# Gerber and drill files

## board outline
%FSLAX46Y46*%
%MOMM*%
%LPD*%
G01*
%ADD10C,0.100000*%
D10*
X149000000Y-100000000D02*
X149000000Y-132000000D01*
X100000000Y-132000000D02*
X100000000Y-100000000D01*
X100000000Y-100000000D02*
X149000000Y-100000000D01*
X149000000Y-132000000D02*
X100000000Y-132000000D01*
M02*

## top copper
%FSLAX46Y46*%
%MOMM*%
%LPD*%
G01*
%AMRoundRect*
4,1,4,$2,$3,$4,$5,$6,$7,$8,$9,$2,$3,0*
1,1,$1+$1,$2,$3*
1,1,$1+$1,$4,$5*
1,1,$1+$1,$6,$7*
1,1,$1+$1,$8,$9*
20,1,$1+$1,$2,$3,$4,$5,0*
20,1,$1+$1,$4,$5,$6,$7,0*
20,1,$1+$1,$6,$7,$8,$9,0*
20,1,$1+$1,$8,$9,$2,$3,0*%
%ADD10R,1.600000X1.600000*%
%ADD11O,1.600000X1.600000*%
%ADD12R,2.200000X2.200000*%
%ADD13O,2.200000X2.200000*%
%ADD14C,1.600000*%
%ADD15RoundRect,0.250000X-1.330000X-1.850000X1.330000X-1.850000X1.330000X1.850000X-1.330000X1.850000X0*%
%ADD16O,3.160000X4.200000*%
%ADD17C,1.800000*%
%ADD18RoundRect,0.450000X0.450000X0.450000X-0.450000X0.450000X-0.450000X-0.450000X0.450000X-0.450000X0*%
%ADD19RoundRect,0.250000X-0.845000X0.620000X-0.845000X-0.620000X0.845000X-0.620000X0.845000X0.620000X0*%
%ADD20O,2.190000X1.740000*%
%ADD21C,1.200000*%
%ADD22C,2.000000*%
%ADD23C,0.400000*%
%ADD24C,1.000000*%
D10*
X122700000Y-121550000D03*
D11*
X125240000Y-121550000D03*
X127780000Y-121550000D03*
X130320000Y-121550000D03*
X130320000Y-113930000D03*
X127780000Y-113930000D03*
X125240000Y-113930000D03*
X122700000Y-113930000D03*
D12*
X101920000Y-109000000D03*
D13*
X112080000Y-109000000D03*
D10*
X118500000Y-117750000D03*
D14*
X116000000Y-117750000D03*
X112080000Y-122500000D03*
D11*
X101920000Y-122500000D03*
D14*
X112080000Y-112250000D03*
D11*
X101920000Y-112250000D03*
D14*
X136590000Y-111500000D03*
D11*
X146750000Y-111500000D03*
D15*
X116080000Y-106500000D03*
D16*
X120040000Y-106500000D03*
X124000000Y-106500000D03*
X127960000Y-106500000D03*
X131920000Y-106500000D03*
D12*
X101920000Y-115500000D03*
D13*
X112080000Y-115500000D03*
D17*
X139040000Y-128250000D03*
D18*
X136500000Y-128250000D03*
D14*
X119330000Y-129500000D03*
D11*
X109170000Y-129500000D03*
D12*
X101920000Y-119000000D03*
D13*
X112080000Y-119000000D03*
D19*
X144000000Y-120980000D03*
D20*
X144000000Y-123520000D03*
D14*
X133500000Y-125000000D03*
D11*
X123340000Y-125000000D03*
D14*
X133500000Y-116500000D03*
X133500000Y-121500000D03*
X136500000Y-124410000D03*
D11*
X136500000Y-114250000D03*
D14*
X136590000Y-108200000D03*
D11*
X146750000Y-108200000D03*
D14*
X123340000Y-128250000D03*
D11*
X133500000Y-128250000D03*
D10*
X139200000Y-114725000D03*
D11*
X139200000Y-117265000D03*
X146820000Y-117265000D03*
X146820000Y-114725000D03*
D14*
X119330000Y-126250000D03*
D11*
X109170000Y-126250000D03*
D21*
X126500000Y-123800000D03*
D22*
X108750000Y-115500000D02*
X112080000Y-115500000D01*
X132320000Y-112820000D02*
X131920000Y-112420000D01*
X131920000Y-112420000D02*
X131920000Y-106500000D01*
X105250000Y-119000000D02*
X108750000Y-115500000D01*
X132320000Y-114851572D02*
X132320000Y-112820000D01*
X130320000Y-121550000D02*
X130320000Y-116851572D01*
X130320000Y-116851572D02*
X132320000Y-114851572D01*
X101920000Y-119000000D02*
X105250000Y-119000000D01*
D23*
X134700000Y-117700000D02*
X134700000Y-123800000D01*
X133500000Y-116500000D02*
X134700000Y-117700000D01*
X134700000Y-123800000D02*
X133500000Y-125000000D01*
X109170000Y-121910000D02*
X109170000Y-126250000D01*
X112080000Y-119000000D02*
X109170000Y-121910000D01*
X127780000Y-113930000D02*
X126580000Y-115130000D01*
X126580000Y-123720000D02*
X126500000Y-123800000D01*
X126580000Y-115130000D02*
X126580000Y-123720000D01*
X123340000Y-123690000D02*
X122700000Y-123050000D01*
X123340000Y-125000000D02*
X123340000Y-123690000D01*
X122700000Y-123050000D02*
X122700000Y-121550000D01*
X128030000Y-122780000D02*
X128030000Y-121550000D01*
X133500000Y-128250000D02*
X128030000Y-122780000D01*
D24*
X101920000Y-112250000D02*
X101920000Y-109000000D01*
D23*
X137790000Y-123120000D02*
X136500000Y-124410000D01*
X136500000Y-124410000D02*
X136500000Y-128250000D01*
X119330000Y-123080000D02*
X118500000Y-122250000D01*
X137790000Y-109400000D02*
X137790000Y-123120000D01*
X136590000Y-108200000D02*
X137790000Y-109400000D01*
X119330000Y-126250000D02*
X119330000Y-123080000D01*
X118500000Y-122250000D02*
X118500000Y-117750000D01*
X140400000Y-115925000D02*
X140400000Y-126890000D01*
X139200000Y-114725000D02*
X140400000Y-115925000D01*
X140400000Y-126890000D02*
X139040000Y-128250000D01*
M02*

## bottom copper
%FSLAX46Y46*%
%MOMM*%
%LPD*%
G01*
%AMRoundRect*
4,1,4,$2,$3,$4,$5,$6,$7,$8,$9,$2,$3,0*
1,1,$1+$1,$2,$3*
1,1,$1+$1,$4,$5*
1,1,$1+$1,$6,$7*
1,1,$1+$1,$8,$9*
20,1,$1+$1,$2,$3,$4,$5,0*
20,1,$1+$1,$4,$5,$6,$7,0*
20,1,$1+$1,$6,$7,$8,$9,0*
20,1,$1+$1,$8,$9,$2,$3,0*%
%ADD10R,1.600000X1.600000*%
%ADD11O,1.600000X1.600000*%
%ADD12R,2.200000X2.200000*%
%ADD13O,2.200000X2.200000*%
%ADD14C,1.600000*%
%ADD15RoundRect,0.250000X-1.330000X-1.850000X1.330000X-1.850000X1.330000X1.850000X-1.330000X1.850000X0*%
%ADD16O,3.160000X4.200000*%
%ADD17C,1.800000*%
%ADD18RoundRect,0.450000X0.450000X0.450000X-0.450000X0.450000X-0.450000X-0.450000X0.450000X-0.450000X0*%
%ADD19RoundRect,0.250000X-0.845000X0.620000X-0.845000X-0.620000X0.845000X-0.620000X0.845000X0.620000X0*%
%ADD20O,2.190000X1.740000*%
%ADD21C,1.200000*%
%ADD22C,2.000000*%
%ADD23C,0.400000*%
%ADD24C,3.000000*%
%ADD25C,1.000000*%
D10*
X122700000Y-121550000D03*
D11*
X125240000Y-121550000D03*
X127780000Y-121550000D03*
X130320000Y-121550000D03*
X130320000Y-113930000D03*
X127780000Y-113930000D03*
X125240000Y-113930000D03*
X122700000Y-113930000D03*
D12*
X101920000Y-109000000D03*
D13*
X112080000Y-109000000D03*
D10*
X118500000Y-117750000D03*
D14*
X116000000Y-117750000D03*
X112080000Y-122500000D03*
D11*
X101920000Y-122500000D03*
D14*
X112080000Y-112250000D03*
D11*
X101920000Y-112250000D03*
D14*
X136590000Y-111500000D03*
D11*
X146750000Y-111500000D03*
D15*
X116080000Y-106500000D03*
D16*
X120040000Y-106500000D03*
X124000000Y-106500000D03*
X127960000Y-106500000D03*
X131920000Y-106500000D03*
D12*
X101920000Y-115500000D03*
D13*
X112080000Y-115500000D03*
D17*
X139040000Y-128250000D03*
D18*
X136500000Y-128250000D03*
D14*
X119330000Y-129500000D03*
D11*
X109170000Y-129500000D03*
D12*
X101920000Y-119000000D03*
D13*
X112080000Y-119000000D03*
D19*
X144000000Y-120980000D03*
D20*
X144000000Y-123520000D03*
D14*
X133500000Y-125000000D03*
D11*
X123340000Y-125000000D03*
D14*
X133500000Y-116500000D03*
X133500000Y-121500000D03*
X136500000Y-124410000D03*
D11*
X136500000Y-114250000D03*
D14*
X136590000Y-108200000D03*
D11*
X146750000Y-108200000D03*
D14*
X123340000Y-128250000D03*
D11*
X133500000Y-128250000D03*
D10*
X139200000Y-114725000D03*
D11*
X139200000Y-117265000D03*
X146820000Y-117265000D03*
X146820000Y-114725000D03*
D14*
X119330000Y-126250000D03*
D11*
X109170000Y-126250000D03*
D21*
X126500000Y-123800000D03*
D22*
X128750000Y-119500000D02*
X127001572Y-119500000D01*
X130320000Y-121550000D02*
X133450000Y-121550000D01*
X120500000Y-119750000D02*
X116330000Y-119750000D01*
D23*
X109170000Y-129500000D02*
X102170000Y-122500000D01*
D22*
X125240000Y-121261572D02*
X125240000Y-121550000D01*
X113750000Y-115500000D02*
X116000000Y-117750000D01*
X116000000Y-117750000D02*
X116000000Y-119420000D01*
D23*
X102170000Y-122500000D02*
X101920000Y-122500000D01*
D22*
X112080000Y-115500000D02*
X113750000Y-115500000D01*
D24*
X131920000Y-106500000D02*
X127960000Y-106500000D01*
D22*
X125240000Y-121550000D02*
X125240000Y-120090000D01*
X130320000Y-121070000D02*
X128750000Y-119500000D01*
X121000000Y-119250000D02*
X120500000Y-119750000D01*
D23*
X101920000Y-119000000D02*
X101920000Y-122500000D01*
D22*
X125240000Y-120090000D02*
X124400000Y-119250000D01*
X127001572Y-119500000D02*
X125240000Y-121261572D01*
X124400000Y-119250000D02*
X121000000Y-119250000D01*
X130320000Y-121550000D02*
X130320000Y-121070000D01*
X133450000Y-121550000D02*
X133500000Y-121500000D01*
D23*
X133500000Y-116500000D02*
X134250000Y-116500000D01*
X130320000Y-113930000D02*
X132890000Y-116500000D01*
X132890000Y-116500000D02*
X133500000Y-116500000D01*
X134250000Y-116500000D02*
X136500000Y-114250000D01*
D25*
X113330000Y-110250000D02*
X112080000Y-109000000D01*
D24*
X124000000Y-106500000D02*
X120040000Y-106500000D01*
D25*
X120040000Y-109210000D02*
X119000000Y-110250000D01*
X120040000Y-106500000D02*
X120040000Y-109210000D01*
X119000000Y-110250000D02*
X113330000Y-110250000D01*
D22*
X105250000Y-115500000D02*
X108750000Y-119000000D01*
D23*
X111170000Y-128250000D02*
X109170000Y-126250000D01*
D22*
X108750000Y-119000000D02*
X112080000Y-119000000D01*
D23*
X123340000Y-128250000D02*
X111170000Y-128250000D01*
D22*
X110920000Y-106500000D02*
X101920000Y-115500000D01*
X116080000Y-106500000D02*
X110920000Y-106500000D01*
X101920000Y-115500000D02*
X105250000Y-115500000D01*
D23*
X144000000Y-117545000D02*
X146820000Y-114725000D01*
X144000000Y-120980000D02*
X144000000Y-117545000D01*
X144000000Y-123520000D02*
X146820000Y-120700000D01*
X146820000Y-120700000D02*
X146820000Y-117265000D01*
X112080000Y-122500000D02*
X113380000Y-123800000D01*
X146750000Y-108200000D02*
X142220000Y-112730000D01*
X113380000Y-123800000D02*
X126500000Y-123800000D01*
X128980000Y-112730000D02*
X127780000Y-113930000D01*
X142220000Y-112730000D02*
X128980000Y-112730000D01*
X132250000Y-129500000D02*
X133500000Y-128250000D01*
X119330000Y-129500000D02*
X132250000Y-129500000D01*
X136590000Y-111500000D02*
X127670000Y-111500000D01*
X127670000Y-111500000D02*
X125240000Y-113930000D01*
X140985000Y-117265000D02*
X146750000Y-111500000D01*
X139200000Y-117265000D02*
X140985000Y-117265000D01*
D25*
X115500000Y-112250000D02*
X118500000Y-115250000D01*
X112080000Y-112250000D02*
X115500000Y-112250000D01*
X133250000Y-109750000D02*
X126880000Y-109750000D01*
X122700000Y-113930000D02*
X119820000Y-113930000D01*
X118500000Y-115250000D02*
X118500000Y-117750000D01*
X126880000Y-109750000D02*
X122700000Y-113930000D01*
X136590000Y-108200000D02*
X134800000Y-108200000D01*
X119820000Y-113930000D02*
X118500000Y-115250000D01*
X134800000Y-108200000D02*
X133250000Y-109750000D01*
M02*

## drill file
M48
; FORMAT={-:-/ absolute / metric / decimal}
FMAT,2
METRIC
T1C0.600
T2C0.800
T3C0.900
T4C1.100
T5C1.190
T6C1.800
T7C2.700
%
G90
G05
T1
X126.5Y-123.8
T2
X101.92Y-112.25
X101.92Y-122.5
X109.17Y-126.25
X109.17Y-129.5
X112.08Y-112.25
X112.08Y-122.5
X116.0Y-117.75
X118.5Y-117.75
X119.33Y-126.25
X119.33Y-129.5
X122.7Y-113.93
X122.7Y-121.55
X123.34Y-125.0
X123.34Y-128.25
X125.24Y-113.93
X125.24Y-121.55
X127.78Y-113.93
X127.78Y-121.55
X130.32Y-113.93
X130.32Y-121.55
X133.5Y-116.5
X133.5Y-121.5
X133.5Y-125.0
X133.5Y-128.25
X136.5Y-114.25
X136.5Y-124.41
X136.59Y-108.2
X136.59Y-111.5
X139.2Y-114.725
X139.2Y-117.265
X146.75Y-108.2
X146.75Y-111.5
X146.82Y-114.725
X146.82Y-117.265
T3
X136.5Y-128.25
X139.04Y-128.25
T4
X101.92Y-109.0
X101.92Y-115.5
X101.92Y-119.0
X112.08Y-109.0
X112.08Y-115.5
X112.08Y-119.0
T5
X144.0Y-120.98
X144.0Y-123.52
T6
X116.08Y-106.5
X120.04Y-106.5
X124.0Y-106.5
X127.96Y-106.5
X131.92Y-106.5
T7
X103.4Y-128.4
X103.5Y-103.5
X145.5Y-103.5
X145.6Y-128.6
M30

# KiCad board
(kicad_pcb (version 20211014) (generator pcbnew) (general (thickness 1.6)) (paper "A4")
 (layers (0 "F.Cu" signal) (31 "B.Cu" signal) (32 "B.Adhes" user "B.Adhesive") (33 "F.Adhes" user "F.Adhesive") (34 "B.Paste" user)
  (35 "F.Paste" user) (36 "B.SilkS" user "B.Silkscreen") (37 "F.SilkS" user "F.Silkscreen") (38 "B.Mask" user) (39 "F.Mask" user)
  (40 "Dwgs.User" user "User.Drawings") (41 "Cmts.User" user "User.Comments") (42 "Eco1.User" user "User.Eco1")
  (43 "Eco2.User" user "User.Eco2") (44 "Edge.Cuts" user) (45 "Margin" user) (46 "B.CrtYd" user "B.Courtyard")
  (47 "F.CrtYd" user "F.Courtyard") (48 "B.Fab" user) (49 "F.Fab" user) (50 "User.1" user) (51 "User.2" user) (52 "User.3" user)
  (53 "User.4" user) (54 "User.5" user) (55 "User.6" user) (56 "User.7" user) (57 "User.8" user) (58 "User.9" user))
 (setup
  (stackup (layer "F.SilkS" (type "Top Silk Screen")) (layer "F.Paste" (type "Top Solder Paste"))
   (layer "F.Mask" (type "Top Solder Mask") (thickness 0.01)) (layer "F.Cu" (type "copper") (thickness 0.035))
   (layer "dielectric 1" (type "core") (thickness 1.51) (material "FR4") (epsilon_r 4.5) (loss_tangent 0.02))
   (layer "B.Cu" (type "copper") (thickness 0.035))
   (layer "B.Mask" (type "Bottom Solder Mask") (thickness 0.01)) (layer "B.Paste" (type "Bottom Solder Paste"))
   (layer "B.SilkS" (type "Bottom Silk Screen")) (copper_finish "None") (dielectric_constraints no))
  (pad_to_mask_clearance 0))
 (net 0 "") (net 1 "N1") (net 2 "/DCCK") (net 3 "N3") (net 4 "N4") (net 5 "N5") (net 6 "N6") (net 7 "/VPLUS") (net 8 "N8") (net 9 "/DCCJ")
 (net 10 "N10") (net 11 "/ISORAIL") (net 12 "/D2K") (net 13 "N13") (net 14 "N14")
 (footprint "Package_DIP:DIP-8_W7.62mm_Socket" (layer "F.Cu") (at 122.7 121.55 90)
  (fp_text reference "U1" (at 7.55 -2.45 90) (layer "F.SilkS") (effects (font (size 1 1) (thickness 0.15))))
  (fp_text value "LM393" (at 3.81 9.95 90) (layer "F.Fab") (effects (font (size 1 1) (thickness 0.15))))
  (pad "1" thru_hole rect (at 0 0 90) (size 1.6 1.6) (drill 0.8) (layers *.Cu *.Mask) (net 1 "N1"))
  (pad "2" thru_hole oval (at 0 2.54 90) (size 1.6 1.6) (drill 0.8) (layers *.Cu *.Mask) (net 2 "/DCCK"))
  (pad "3" thru_hole oval (at 0 5.08 90) (size 1.6 1.6) (drill 0.8) (layers *.Cu *.Mask) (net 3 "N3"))
  (pad "4" thru_hole oval (at 0 7.62 90) (size 1.6 1.6) (drill 0.8) (layers *.Cu *.Mask) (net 2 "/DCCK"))
  (pad "5" thru_hole oval (at 7.62 7.62 90) (size 1.6 1.6) (drill 0.8) (layers *.Cu *.Mask) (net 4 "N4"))
  (pad "6" thru_hole oval (at 7.62 5.08 90) (size 1.6 1.6) (drill 0.8) (layers *.Cu *.Mask) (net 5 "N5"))
  (pad "7" thru_hole oval (at 7.62 2.54 90) (size 1.6 1.6) (drill 0.8) (layers *.Cu *.Mask) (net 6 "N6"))
  (pad "8" thru_hole oval (at 7.62 0 90) (size 1.6 1.6) (drill 0.8) (layers *.Cu *.Mask) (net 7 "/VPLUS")))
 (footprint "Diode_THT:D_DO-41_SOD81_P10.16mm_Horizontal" (layer "F.Cu") (at 101.92 109)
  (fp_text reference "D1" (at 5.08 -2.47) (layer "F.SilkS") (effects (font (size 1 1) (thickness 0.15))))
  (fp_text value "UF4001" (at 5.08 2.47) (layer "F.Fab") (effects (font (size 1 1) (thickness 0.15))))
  (pad "1" thru_hole rect (at 0 0) (size 2.2 2.2) (drill 1.1) (layers *.Cu *.Mask) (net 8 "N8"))
  (pad "2" thru_hole oval (at 10.16 0) (size 2.2 2.2) (drill 1.1) (layers *.Cu *.Mask) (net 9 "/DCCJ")))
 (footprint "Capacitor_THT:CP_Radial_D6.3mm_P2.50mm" (layer "F.Cu") (at 118.5 117.75 180)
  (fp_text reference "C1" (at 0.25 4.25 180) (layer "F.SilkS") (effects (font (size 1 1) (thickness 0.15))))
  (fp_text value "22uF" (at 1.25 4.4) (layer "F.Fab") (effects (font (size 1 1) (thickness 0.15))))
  (pad "1" thru_hole rect (at 0 0 180) (size 1.6 1.6) (drill 0.8) (layers *.Cu *.Mask) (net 7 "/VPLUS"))
  (pad "2" thru_hole circle (at 2.5 0 180) (size 1.6 1.6) (drill 0.8) (layers *.Cu *.Mask) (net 2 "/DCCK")))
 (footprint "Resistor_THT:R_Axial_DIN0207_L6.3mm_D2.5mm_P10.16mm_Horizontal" (layer "F.Cu") (at 112.08 122.5 180)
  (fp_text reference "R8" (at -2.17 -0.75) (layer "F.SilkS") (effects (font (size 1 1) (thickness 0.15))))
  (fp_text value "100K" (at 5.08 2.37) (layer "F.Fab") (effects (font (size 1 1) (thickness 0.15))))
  (pad "1" thru_hole circle (at 0 0 180) (size 1.6 1.6) (drill 0.8) (layers *.Cu *.Mask) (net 5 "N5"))
  (pad "2" thru_hole oval (at 10.16 0 180) (size 1.6 1.6) (drill 0.8) (layers *.Cu *.Mask) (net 2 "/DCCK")))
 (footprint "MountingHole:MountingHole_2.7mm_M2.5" (layer "F.Cu") (at 145.5 103.5)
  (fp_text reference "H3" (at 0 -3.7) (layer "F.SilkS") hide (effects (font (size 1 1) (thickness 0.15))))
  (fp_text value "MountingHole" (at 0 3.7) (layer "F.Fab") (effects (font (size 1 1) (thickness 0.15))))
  (pad "" np_thru_hole circle (at 0 0) (size 2.7 2.7) (drill 2.7) (layers *.Cu *.Mask)))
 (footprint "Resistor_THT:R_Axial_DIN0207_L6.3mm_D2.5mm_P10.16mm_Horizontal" (layer "F.Cu") (at 112.08 112.25 180)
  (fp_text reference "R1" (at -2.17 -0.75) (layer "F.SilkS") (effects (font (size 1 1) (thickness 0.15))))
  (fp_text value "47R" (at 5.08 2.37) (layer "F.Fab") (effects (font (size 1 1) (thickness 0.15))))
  (pad "1" thru_hole circle (at 0 0 180) (size 1.6 1.6) (drill 0.8) (layers *.Cu *.Mask) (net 7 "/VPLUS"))
  (pad "2" thru_hole oval (at 10.16 0 180) (size 1.6 1.6) (drill 0.8) (layers *.Cu *.Mask) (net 8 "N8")))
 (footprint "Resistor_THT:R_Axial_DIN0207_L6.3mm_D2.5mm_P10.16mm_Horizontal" (layer "F.Cu") (at 136.59 111.5)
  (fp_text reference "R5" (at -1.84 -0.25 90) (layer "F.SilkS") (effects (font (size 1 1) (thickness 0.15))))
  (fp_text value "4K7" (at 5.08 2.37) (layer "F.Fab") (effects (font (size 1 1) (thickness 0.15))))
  (pad "1" thru_hole circle (at 0 0) (size 1.6 1.6) (drill 0.8) (layers *.Cu *.Mask) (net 6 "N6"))
  (pad "2" thru_hole oval (at 10.16 0) (size 1.6 1.6) (drill 0.8) (layers *.Cu *.Mask) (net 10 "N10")))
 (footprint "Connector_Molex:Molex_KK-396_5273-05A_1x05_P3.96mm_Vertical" (layer "F.Cu") (at 116.08 106.5)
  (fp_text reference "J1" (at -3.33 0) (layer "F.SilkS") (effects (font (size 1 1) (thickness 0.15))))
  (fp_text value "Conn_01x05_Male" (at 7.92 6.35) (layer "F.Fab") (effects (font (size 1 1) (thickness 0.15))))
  (pad "1" thru_hole roundrect (at 0 0) (size 3.16 4.2) (drill 1.8) (layers *.Cu *.Mask) (roundrect_rratio 0.079114) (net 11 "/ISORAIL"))
  (pad "2" thru_hole oval (at 3.96 0) (size 3.16 4.2) (drill 1.8) (layers *.Cu *.Mask) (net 9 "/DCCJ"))
  (pad "3" thru_hole oval (at 7.92 0) (size 3.16 4.2) (drill 1.8) (layers *.Cu *.Mask) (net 9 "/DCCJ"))
  (pad "4" thru_hole oval (at 11.88 0) (size 3.16 4.2) (drill 1.8) (layers *.Cu *.Mask) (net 2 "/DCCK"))
  (pad "5" thru_hole oval (at 15.84 0) (size 3.16 4.2) (drill 1.8) (layers *.Cu *.Mask) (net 2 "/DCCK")))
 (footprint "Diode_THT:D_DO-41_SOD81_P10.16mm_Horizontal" (layer "F.Cu") (at 101.92 115.5)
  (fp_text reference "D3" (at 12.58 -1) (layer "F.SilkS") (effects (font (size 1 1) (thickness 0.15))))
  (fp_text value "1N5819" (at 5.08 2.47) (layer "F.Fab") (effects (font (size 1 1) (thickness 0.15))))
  (pad "1" thru_hole rect (at 0 0) (size 2.2 2.2) (drill 1.1) (layers *.Cu *.Mask) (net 11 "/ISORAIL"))
  (pad "2" thru_hole oval (at 10.16 0) (size 2.2 2.2) (drill 1.1) (layers *.Cu *.Mask) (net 2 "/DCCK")))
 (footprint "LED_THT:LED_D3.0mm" (layer "F.Cu") (at 139.04 128.25 180)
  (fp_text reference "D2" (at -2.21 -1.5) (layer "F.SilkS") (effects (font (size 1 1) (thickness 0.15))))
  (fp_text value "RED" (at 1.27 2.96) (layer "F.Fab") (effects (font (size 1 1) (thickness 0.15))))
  (pad "1" thru_hole circle (at 0 0 180) (size 1.8 1.8) (drill 0.9) (layers *.Cu *.Mask) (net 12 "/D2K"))
  (pad "2" thru_hole roundrect (at 2.54 0 180) (size 1.8 1.8) (drill 0.9) (layers *.Cu *.Mask) (roundrect_rratio 0.25) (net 7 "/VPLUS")))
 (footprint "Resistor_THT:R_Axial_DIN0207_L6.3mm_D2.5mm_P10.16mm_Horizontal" (layer "F.Cu") (at 119.33 129.5 180)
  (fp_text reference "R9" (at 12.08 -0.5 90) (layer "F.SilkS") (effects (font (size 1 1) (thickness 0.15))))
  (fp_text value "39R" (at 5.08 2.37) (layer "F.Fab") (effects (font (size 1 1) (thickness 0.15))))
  (pad "1" thru_hole circle (at 0 0 180) (size 1.6 1.6) (drill 0.8) (layers *.Cu *.Mask) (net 3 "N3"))
  (pad "2" thru_hole oval (at 10.16 0 180) (size 1.6 1.6) (drill 0.8) (layers *.Cu *.Mask) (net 2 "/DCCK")))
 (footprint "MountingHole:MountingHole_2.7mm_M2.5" (layer "F.Cu") (at 103.5 103.5)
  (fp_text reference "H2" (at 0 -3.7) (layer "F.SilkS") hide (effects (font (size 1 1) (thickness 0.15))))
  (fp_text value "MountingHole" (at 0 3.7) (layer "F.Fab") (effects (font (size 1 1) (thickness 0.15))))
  (pad "" np_thru_hole circle (at 0 0) (size 2.7 2.7) (drill 2.7) (layers *.Cu *.Mask)))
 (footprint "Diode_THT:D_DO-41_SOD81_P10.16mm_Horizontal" (layer "F.Cu") (at 101.92 119)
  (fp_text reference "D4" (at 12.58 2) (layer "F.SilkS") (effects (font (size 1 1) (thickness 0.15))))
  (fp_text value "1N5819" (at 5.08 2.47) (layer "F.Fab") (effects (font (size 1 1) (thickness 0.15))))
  (pad "1" thru_hole rect (at 0 0) (size 2.2 2.2) (drill 1.1) (layers *.Cu *.Mask) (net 2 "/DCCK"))
  (pad "2" thru_hole oval (at 10.16 0) (size 2.2 2.2) (drill 1.1) (layers *.Cu *.Mask) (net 11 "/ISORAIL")))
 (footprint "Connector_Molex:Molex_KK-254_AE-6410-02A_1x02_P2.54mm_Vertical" (layer "F.Cu") (at 144 120.98 -90)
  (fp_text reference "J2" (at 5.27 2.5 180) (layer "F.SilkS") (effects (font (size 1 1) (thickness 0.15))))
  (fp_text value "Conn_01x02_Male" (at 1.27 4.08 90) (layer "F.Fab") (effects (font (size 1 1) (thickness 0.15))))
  (pad "1" thru_hole roundrect (at 0 0 270) (size 1.74 2.19) (drill 1.19) (layers *.Cu *.Mask) (roundrect_rratio 0.143678) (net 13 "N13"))
  (pad "2" thru_hole oval (at 2.54 0 270) (size 1.74 2.19) (drill 1.19) (layers *.Cu *.Mask) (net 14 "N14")))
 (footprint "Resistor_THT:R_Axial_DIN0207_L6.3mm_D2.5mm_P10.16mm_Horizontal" (layer "F.Cu") (at 133.5 125 180)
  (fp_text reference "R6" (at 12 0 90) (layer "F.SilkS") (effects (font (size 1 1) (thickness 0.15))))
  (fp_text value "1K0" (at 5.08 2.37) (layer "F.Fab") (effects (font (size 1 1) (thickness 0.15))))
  (pad "1" thru_hole circle (at 0 0 180) (size 1.6 1.6) (drill 0.8) (layers *.Cu *.Mask) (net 4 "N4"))
  (pad "2" thru_hole oval (at 10.16 0 180) (size 1.6 1.6) (drill 0.8) (layers *.Cu *.Mask) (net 1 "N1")))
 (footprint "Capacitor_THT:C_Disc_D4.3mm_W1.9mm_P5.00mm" (layer "F.Cu") (at 133.5 116.5 -90)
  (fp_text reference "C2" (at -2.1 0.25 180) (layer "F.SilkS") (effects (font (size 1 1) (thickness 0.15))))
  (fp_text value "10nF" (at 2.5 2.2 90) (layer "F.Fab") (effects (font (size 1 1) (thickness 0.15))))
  (pad "1" thru_hole circle (at 0 0 270) (size 1.6 1.6) (drill 0.8) (layers *.Cu *.Mask) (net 4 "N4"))
  (pad "2" thru_hole circle (at 5 0 270) (size 1.6 1.6) (drill 0.8) (layers *.Cu *.Mask) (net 2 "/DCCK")))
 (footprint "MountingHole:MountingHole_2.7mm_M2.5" (layer "F.Cu") (at 145.6 128.6)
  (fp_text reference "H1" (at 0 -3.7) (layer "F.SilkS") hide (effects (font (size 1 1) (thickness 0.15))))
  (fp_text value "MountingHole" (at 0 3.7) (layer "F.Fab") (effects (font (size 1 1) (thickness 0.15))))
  (pad "" np_thru_hole circle (at 0 0) (size 2.7 2.7) (drill 2.7) (layers *.Cu *.Mask)))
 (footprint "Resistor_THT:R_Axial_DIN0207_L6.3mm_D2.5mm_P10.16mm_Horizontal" (layer "F.Cu") (at 136.5 124.41 90)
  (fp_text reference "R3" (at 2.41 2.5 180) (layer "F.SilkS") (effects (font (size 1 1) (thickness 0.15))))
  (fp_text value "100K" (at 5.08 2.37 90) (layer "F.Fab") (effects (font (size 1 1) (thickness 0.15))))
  (pad "1" thru_hole circle (at 0 0 90) (size 1.6 1.6) (drill 0.8) (layers *.Cu *.Mask) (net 7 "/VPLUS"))
  (pad "2" thru_hole oval (at 10.16 0 90) (size 1.6 1.6) (drill 0.8) (layers *.Cu *.Mask) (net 4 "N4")))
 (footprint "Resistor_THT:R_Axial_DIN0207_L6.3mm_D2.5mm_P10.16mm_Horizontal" (layer "F.Cu") (at 136.59 108.2)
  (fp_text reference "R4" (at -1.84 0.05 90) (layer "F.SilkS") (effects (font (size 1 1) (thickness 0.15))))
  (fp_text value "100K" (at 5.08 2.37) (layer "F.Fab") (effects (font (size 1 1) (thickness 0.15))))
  (pad "1" thru_hole circle (at 0 0) (size 1.6 1.6) (drill 0.8) (layers *.Cu *.Mask) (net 7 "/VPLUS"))
  (pad "2" thru_hole oval (at 10.16 0) (size 1.6 1.6) (drill 0.8) (layers *.Cu *.Mask) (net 5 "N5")))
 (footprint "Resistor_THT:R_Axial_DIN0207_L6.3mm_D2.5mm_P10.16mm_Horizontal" (layer "F.Cu") (at 123.34 128.25)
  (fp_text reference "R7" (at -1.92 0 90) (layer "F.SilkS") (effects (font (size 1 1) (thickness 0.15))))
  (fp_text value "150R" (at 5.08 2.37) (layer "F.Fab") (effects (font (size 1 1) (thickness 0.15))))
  (pad "1" thru_hole circle (at 0 0) (size 1.6 1.6) (drill 0.8) (layers *.Cu *.Mask) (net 11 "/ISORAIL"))
  (pad "2" thru_hole oval (at 10.16 0) (size 1.6 1.6) (drill 0.8) (layers *.Cu *.Mask) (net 3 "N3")))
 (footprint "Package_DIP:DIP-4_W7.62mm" (layer "F.Cu") (at 139.2 114.725)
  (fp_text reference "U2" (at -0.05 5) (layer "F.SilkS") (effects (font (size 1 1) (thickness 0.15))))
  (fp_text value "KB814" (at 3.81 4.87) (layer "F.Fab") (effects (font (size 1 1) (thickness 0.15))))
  (pad "1" thru_hole rect (at 0 0) (size 1.6 1.6) (drill 0.8) (layers *.Cu *.Mask) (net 12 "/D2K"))
  (pad "2" thru_hole oval (at 0 2.54) (size 1.6 1.6) (drill 0.8) (layers *.Cu *.Mask) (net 10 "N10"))
  (pad "3" thru_hole oval (at 7.62 2.54) (size 1.6 1.6) (drill 0.8) (layers *.Cu *.Mask) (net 14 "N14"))
  (pad "4" thru_hole oval (at 7.62 0) (size 1.6 1.6) (drill 0.8) (layers *.Cu *.Mask) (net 13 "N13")))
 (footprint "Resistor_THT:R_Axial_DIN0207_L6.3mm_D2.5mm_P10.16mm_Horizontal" (layer "F.Cu") (at 119.33 126.25 180)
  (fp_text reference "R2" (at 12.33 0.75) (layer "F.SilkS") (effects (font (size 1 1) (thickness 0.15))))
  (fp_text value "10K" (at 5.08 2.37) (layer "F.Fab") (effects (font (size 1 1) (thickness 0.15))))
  (pad "1" thru_hole circle (at 0 0 180) (size 1.6 1.6) (drill 0.8) (layers *.Cu *.Mask) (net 7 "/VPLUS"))
  (pad "2" thru_hole oval (at 10.16 0 180) (size 1.6 1.6) (drill 0.8) (layers *.Cu *.Mask) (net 11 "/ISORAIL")))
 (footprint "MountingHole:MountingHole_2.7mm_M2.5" (layer "F.Cu") (at 103.4 128.4)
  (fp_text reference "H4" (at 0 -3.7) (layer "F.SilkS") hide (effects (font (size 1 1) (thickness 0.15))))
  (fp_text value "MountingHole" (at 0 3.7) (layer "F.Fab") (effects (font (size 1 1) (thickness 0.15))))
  (pad "" np_thru_hole circle (at 0 0) (size 2.7 2.7) (drill 2.7) (layers *.Cu *.Mask)))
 (gr_line (start 149 100) (end 149 132) (layer "Edge.Cuts") (width 0.1))
 (gr_line (start 100 132) (end 100 100) (layer "Edge.Cuts") (width 0.1))
 (gr_line (start 100 100) (end 149 100) (layer "Edge.Cuts") (width 0.1))
 (gr_line (start 149 132) (end 100 132) (layer "Edge.Cuts") (width 0.1))
 (segment (start 108.75 115.5) (end 112.08 115.5) (width 2) (layer "F.Cu") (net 2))
 (segment (start 132.32 112.82) (end 131.92 112.42) (width 2) (layer "F.Cu") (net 2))
 (segment (start 131.92 112.42) (end 131.92 106.5) (width 2) (layer "F.Cu") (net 2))
 (segment (start 105.25 119) (end 108.75 115.5) (width 2) (layer "F.Cu") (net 2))
 (segment (start 132.32 114.851572) (end 132.32 112.82) (width 2) (layer "F.Cu") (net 2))
 (segment (start 130.32 121.55) (end 130.32 116.851572) (width 2) (layer "F.Cu") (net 2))
 (segment (start 130.32 116.851572) (end 132.32 114.851572) (width 2) (layer "F.Cu") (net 2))
 (segment (start 101.92 119) (end 105.25 119) (width 2) (layer "F.Cu") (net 2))
 (segment (start 128.75 119.5) (end 127.001572 119.5) (width 2) (layer "B.Cu") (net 2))
 (segment (start 130.32 121.55) (end 133.45 121.55) (width 2) (layer "B.Cu") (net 2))
 (segment (start 120.5 119.75) (end 116.33 119.75) (width 2) (layer "B.Cu") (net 2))
 (segment (start 109.17 129.5) (end 102.17 122.5) (width 0.4) (layer "B.Cu") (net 2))
 (segment (start 125.24 121.261572) (end 125.24 121.55) (width 2) (layer "B.Cu") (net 2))
 (segment (start 113.75 115.5) (end 116 117.75) (width 2) (layer "B.Cu") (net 2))
 (segment (start 116 117.75) (end 116 119.42) (width 2) (layer "B.Cu") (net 2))
 (segment (start 102.17 122.5) (end 101.92 122.5) (width 0.4) (layer "B.Cu") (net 2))
 (segment (start 112.08 115.5) (end 113.75 115.5) (width 2) (layer "B.Cu") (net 2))
 (segment (start 131.92 106.5) (end 127.96 106.5) (width 3) (layer "B.Cu") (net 2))
 (segment (start 125.24 121.55) (end 125.24 120.09) (width 2) (layer "B.Cu") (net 2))
 (segment (start 130.32 121.07) (end 128.75 119.5) (width 2) (layer "B.Cu") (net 2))
 (segment (start 121 119.25) (end 120.5 119.75) (width 2) (layer "B.Cu") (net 2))
 (segment (start 101.92 119) (end 101.92 122.5) (width 0.4) (layer "B.Cu") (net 2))
 (segment (start 125.24 120.09) (end 124.4 119.25) (width 2) (layer "B.Cu") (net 2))
 (segment (start 127.001572 119.5) (end 125.24 121.261572) (width 2) (layer "B.Cu") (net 2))
 (segment (start 124.4 119.25) (end 121 119.25) (width 2) (layer "B.Cu") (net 2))
 (segment (start 130.32 121.55) (end 130.32 121.07) (width 2) (layer "B.Cu") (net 2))
 (segment (start 133.45 121.55) (end 133.5 121.5) (width 2) (layer "B.Cu") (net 2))
 (segment (start 134.7 117.7) (end 134.7 123.8) (width 0.4) (layer "F.Cu") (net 4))
 (segment (start 133.5 116.5) (end 134.7 117.7) (width 0.4) (layer "F.Cu") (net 4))
 (segment (start 134.7 123.8) (end 133.5 125) (width 0.4) (layer "F.Cu") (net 4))
 (segment (start 133.5 116.5) (end 134.25 116.5) (width 0.4) (layer "B.Cu") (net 4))
 (segment (start 130.32 113.93) (end 132.89 116.5) (width 0.4) (layer "B.Cu") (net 4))
 (segment (start 132.89 116.5) (end 133.5 116.5) (width 0.4) (layer "B.Cu") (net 4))
 (segment (start 134.25 116.5) (end 136.5 114.25) (width 0.4) (layer "B.Cu") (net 4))
 (segment (start 113.33 110.25) (end 112.08 109) (width 1) (layer "B.Cu") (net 9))
 (segment (start 124 106.5) (end 120.04 106.5) (width 3) (layer "B.Cu") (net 9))
 (segment (start 120.04 109.21) (end 119 110.25) (width 1) (layer "B.Cu") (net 9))
 (segment (start 120.04 106.5) (end 120.04 109.21) (width 1) (layer "B.Cu") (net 9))
 (segment (start 119 110.25) (end 113.33 110.25) (width 1) (layer "B.Cu") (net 9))
 (segment (start 109.17 121.91) (end 109.17 126.25) (width 0.4) (layer "F.Cu") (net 11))
 (segment (start 112.08 119) (end 109.17 121.91) (width 0.4) (layer "F.Cu") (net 11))
 (segment (start 105.25 115.5) (end 108.75 119) (width 2) (layer "B.Cu") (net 11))
 (segment (start 111.17 128.25) (end 109.17 126.25) (width 0.4) (layer "B.Cu") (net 11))
 (segment (start 108.75 119) (end 112.08 119) (width 2) (layer "B.Cu") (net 11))
 (segment (start 123.34 128.25) (end 111.17 128.25) (width 0.4) (layer "B.Cu") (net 11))
 (segment (start 110.92 106.5) (end 101.92 115.5) (width 2) (layer "B.Cu") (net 11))
 (segment (start 116.08 106.5) (end 110.92 106.5) (width 2) (layer "B.Cu") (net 11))
 (segment (start 101.92 115.5) (end 105.25 115.5) (width 2) (layer "B.Cu") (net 11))
 (segment (start 144 117.545) (end 146.82 114.725) (width 0.4) (layer "B.Cu") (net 13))
 (segment (start 144 120.98) (end 144 117.545) (width 0.4) (layer "B.Cu") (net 13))
 (segment (start 144 123.52) (end 146.82 120.7) (width 0.4) (layer "B.Cu") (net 14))
 (segment (start 146.82 120.7) (end 146.82 117.265) (width 0.4) (layer "B.Cu") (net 14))
 (segment (start 127.78 113.93) (end 126.58 115.13) (width 0.4) (layer "F.Cu") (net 5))
 (segment (start 126.58 123.72) (end 126.5 123.8) (width 0.4) (layer "F.Cu") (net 5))
 (segment (start 126.58 115.13) (end 126.58 123.72) (width 0.4) (layer "F.Cu") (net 5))
 (via (at 126.5 123.8) (size 1.2) (drill 0.6) (layers "F.Cu" "B.Cu") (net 5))
 (segment (start 112.08 122.5) (end 113.38 123.8) (width 0.4) (layer "B.Cu") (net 5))
 (segment (start 146.75 108.2) (end 142.22 112.73) (width 0.4) (layer "B.Cu") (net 5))
 (segment (start 113.38 123.8) (end 126.5 123.8) (width 0.4) (layer "B.Cu") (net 5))
 (segment (start 128.98 112.73) (end 127.78 113.93) (width 0.4) (layer "B.Cu") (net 5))
 (segment (start 142.22 112.73) (end 128.98 112.73) (width 0.4) (layer "B.Cu") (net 5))
 (segment (start 123.34 123.69) (end 122.7 123.05) (width 0.4) (layer "F.Cu") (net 1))
 (segment (start 123.34 125) (end 123.34 123.69) (width 0.4) (layer "F.Cu") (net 1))
 (segment (start 122.7 123.05) (end 122.7 121.55) (width 0.4) (layer "F.Cu") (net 1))
 (segment (start 128.03 122.78) (end 128.03 121.55) (width 0.4) (layer "F.Cu") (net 3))
 (segment (start 133.5 128.25) (end 128.03 122.78) (width 0.4) (layer "F.Cu") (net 3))
 (segment (start 132.25 129.5) (end 133.5 128.25) (width 0.4) (layer "B.Cu") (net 3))
 (segment (start 119.33 129.5) (end 132.25 129.5) (width 0.4) (layer "B.Cu") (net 3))
 (segment (start 136.59 111.5) (end 127.67 111.5) (width 0.4) (layer "B.Cu") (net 6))
 (segment (start 127.67 111.5) (end 125.24 113.93) (width 0.4) (layer "B.Cu") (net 6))
 (segment (start 101.92 112.25) (end 101.92 109) (width 1) (layer "F.Cu") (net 8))
 (segment (start 140.985 117.265) (end 146.75 111.5) (width 0.4) (layer "B.Cu") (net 10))
 (segment (start 139.2 117.265) (end 140.985 117.265) (width 0.4) (layer "B.Cu") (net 10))
 (segment (start 137.79 123.12) (end 136.5 124.41) (width 0.4) (layer "F.Cu") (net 7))
 (segment (start 136.5 124.41) (end 136.5 128.25) (width 0.4) (layer "F.Cu") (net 7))
 (segment (start 119.33 123.08) (end 118.5 122.25) (width 0.4) (layer "F.Cu") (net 7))
 (segment (start 137.79 109.4) (end 137.79 123.12) (width 0.4) (layer "F.Cu") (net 7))
 (segment (start 136.59 108.2) (end 137.79 109.4) (width 0.4) (layer "F.Cu") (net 7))
 (segment (start 119.33 126.25) (end 119.33 123.08) (width 0.4) (layer "F.Cu") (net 7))
 (segment (start 118.5 122.25) (end 118.5 117.75) (width 0.4) (layer "F.Cu") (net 7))
 (segment (start 115.5 112.25) (end 118.5 115.25) (width 1) (layer "B.Cu") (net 7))
 (segment (start 112.08 112.25) (end 115.5 112.25) (width 1) (layer "B.Cu") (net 7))
 (segment (start 133.25 109.75) (end 126.88 109.75) (width 1) (layer "B.Cu") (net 7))
 (segment (start 122.7 113.93) (end 119.82 113.93) (width 1) (layer "B.Cu") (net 7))
 (segment (start 118.5 115.25) (end 118.5 117.75) (width 1) (layer "B.Cu") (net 7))
 (segment (start 126.88 109.75) (end 122.7 113.93) (width 1) (layer "B.Cu") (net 7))
 (segment (start 136.59 108.2) (end 134.8 108.2) (width 1) (layer "B.Cu") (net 7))
 (segment (start 119.82 113.93) (end 118.5 115.25) (width 1) (layer "B.Cu") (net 7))
 (segment (start 134.8 108.2) (end 133.25 109.75) (width 1) (layer "B.Cu") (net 7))
 (segment (start 140.4 115.925) (end 140.4 126.89) (width 0.4) (layer "F.Cu") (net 12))
 (segment (start 139.2 114.725) (end 140.4 115.925) (width 0.4) (layer "F.Cu") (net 12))
 (segment (start 140.4 126.89) (end 139.04 128.25) (width 0.4) (layer "F.Cu") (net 12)))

